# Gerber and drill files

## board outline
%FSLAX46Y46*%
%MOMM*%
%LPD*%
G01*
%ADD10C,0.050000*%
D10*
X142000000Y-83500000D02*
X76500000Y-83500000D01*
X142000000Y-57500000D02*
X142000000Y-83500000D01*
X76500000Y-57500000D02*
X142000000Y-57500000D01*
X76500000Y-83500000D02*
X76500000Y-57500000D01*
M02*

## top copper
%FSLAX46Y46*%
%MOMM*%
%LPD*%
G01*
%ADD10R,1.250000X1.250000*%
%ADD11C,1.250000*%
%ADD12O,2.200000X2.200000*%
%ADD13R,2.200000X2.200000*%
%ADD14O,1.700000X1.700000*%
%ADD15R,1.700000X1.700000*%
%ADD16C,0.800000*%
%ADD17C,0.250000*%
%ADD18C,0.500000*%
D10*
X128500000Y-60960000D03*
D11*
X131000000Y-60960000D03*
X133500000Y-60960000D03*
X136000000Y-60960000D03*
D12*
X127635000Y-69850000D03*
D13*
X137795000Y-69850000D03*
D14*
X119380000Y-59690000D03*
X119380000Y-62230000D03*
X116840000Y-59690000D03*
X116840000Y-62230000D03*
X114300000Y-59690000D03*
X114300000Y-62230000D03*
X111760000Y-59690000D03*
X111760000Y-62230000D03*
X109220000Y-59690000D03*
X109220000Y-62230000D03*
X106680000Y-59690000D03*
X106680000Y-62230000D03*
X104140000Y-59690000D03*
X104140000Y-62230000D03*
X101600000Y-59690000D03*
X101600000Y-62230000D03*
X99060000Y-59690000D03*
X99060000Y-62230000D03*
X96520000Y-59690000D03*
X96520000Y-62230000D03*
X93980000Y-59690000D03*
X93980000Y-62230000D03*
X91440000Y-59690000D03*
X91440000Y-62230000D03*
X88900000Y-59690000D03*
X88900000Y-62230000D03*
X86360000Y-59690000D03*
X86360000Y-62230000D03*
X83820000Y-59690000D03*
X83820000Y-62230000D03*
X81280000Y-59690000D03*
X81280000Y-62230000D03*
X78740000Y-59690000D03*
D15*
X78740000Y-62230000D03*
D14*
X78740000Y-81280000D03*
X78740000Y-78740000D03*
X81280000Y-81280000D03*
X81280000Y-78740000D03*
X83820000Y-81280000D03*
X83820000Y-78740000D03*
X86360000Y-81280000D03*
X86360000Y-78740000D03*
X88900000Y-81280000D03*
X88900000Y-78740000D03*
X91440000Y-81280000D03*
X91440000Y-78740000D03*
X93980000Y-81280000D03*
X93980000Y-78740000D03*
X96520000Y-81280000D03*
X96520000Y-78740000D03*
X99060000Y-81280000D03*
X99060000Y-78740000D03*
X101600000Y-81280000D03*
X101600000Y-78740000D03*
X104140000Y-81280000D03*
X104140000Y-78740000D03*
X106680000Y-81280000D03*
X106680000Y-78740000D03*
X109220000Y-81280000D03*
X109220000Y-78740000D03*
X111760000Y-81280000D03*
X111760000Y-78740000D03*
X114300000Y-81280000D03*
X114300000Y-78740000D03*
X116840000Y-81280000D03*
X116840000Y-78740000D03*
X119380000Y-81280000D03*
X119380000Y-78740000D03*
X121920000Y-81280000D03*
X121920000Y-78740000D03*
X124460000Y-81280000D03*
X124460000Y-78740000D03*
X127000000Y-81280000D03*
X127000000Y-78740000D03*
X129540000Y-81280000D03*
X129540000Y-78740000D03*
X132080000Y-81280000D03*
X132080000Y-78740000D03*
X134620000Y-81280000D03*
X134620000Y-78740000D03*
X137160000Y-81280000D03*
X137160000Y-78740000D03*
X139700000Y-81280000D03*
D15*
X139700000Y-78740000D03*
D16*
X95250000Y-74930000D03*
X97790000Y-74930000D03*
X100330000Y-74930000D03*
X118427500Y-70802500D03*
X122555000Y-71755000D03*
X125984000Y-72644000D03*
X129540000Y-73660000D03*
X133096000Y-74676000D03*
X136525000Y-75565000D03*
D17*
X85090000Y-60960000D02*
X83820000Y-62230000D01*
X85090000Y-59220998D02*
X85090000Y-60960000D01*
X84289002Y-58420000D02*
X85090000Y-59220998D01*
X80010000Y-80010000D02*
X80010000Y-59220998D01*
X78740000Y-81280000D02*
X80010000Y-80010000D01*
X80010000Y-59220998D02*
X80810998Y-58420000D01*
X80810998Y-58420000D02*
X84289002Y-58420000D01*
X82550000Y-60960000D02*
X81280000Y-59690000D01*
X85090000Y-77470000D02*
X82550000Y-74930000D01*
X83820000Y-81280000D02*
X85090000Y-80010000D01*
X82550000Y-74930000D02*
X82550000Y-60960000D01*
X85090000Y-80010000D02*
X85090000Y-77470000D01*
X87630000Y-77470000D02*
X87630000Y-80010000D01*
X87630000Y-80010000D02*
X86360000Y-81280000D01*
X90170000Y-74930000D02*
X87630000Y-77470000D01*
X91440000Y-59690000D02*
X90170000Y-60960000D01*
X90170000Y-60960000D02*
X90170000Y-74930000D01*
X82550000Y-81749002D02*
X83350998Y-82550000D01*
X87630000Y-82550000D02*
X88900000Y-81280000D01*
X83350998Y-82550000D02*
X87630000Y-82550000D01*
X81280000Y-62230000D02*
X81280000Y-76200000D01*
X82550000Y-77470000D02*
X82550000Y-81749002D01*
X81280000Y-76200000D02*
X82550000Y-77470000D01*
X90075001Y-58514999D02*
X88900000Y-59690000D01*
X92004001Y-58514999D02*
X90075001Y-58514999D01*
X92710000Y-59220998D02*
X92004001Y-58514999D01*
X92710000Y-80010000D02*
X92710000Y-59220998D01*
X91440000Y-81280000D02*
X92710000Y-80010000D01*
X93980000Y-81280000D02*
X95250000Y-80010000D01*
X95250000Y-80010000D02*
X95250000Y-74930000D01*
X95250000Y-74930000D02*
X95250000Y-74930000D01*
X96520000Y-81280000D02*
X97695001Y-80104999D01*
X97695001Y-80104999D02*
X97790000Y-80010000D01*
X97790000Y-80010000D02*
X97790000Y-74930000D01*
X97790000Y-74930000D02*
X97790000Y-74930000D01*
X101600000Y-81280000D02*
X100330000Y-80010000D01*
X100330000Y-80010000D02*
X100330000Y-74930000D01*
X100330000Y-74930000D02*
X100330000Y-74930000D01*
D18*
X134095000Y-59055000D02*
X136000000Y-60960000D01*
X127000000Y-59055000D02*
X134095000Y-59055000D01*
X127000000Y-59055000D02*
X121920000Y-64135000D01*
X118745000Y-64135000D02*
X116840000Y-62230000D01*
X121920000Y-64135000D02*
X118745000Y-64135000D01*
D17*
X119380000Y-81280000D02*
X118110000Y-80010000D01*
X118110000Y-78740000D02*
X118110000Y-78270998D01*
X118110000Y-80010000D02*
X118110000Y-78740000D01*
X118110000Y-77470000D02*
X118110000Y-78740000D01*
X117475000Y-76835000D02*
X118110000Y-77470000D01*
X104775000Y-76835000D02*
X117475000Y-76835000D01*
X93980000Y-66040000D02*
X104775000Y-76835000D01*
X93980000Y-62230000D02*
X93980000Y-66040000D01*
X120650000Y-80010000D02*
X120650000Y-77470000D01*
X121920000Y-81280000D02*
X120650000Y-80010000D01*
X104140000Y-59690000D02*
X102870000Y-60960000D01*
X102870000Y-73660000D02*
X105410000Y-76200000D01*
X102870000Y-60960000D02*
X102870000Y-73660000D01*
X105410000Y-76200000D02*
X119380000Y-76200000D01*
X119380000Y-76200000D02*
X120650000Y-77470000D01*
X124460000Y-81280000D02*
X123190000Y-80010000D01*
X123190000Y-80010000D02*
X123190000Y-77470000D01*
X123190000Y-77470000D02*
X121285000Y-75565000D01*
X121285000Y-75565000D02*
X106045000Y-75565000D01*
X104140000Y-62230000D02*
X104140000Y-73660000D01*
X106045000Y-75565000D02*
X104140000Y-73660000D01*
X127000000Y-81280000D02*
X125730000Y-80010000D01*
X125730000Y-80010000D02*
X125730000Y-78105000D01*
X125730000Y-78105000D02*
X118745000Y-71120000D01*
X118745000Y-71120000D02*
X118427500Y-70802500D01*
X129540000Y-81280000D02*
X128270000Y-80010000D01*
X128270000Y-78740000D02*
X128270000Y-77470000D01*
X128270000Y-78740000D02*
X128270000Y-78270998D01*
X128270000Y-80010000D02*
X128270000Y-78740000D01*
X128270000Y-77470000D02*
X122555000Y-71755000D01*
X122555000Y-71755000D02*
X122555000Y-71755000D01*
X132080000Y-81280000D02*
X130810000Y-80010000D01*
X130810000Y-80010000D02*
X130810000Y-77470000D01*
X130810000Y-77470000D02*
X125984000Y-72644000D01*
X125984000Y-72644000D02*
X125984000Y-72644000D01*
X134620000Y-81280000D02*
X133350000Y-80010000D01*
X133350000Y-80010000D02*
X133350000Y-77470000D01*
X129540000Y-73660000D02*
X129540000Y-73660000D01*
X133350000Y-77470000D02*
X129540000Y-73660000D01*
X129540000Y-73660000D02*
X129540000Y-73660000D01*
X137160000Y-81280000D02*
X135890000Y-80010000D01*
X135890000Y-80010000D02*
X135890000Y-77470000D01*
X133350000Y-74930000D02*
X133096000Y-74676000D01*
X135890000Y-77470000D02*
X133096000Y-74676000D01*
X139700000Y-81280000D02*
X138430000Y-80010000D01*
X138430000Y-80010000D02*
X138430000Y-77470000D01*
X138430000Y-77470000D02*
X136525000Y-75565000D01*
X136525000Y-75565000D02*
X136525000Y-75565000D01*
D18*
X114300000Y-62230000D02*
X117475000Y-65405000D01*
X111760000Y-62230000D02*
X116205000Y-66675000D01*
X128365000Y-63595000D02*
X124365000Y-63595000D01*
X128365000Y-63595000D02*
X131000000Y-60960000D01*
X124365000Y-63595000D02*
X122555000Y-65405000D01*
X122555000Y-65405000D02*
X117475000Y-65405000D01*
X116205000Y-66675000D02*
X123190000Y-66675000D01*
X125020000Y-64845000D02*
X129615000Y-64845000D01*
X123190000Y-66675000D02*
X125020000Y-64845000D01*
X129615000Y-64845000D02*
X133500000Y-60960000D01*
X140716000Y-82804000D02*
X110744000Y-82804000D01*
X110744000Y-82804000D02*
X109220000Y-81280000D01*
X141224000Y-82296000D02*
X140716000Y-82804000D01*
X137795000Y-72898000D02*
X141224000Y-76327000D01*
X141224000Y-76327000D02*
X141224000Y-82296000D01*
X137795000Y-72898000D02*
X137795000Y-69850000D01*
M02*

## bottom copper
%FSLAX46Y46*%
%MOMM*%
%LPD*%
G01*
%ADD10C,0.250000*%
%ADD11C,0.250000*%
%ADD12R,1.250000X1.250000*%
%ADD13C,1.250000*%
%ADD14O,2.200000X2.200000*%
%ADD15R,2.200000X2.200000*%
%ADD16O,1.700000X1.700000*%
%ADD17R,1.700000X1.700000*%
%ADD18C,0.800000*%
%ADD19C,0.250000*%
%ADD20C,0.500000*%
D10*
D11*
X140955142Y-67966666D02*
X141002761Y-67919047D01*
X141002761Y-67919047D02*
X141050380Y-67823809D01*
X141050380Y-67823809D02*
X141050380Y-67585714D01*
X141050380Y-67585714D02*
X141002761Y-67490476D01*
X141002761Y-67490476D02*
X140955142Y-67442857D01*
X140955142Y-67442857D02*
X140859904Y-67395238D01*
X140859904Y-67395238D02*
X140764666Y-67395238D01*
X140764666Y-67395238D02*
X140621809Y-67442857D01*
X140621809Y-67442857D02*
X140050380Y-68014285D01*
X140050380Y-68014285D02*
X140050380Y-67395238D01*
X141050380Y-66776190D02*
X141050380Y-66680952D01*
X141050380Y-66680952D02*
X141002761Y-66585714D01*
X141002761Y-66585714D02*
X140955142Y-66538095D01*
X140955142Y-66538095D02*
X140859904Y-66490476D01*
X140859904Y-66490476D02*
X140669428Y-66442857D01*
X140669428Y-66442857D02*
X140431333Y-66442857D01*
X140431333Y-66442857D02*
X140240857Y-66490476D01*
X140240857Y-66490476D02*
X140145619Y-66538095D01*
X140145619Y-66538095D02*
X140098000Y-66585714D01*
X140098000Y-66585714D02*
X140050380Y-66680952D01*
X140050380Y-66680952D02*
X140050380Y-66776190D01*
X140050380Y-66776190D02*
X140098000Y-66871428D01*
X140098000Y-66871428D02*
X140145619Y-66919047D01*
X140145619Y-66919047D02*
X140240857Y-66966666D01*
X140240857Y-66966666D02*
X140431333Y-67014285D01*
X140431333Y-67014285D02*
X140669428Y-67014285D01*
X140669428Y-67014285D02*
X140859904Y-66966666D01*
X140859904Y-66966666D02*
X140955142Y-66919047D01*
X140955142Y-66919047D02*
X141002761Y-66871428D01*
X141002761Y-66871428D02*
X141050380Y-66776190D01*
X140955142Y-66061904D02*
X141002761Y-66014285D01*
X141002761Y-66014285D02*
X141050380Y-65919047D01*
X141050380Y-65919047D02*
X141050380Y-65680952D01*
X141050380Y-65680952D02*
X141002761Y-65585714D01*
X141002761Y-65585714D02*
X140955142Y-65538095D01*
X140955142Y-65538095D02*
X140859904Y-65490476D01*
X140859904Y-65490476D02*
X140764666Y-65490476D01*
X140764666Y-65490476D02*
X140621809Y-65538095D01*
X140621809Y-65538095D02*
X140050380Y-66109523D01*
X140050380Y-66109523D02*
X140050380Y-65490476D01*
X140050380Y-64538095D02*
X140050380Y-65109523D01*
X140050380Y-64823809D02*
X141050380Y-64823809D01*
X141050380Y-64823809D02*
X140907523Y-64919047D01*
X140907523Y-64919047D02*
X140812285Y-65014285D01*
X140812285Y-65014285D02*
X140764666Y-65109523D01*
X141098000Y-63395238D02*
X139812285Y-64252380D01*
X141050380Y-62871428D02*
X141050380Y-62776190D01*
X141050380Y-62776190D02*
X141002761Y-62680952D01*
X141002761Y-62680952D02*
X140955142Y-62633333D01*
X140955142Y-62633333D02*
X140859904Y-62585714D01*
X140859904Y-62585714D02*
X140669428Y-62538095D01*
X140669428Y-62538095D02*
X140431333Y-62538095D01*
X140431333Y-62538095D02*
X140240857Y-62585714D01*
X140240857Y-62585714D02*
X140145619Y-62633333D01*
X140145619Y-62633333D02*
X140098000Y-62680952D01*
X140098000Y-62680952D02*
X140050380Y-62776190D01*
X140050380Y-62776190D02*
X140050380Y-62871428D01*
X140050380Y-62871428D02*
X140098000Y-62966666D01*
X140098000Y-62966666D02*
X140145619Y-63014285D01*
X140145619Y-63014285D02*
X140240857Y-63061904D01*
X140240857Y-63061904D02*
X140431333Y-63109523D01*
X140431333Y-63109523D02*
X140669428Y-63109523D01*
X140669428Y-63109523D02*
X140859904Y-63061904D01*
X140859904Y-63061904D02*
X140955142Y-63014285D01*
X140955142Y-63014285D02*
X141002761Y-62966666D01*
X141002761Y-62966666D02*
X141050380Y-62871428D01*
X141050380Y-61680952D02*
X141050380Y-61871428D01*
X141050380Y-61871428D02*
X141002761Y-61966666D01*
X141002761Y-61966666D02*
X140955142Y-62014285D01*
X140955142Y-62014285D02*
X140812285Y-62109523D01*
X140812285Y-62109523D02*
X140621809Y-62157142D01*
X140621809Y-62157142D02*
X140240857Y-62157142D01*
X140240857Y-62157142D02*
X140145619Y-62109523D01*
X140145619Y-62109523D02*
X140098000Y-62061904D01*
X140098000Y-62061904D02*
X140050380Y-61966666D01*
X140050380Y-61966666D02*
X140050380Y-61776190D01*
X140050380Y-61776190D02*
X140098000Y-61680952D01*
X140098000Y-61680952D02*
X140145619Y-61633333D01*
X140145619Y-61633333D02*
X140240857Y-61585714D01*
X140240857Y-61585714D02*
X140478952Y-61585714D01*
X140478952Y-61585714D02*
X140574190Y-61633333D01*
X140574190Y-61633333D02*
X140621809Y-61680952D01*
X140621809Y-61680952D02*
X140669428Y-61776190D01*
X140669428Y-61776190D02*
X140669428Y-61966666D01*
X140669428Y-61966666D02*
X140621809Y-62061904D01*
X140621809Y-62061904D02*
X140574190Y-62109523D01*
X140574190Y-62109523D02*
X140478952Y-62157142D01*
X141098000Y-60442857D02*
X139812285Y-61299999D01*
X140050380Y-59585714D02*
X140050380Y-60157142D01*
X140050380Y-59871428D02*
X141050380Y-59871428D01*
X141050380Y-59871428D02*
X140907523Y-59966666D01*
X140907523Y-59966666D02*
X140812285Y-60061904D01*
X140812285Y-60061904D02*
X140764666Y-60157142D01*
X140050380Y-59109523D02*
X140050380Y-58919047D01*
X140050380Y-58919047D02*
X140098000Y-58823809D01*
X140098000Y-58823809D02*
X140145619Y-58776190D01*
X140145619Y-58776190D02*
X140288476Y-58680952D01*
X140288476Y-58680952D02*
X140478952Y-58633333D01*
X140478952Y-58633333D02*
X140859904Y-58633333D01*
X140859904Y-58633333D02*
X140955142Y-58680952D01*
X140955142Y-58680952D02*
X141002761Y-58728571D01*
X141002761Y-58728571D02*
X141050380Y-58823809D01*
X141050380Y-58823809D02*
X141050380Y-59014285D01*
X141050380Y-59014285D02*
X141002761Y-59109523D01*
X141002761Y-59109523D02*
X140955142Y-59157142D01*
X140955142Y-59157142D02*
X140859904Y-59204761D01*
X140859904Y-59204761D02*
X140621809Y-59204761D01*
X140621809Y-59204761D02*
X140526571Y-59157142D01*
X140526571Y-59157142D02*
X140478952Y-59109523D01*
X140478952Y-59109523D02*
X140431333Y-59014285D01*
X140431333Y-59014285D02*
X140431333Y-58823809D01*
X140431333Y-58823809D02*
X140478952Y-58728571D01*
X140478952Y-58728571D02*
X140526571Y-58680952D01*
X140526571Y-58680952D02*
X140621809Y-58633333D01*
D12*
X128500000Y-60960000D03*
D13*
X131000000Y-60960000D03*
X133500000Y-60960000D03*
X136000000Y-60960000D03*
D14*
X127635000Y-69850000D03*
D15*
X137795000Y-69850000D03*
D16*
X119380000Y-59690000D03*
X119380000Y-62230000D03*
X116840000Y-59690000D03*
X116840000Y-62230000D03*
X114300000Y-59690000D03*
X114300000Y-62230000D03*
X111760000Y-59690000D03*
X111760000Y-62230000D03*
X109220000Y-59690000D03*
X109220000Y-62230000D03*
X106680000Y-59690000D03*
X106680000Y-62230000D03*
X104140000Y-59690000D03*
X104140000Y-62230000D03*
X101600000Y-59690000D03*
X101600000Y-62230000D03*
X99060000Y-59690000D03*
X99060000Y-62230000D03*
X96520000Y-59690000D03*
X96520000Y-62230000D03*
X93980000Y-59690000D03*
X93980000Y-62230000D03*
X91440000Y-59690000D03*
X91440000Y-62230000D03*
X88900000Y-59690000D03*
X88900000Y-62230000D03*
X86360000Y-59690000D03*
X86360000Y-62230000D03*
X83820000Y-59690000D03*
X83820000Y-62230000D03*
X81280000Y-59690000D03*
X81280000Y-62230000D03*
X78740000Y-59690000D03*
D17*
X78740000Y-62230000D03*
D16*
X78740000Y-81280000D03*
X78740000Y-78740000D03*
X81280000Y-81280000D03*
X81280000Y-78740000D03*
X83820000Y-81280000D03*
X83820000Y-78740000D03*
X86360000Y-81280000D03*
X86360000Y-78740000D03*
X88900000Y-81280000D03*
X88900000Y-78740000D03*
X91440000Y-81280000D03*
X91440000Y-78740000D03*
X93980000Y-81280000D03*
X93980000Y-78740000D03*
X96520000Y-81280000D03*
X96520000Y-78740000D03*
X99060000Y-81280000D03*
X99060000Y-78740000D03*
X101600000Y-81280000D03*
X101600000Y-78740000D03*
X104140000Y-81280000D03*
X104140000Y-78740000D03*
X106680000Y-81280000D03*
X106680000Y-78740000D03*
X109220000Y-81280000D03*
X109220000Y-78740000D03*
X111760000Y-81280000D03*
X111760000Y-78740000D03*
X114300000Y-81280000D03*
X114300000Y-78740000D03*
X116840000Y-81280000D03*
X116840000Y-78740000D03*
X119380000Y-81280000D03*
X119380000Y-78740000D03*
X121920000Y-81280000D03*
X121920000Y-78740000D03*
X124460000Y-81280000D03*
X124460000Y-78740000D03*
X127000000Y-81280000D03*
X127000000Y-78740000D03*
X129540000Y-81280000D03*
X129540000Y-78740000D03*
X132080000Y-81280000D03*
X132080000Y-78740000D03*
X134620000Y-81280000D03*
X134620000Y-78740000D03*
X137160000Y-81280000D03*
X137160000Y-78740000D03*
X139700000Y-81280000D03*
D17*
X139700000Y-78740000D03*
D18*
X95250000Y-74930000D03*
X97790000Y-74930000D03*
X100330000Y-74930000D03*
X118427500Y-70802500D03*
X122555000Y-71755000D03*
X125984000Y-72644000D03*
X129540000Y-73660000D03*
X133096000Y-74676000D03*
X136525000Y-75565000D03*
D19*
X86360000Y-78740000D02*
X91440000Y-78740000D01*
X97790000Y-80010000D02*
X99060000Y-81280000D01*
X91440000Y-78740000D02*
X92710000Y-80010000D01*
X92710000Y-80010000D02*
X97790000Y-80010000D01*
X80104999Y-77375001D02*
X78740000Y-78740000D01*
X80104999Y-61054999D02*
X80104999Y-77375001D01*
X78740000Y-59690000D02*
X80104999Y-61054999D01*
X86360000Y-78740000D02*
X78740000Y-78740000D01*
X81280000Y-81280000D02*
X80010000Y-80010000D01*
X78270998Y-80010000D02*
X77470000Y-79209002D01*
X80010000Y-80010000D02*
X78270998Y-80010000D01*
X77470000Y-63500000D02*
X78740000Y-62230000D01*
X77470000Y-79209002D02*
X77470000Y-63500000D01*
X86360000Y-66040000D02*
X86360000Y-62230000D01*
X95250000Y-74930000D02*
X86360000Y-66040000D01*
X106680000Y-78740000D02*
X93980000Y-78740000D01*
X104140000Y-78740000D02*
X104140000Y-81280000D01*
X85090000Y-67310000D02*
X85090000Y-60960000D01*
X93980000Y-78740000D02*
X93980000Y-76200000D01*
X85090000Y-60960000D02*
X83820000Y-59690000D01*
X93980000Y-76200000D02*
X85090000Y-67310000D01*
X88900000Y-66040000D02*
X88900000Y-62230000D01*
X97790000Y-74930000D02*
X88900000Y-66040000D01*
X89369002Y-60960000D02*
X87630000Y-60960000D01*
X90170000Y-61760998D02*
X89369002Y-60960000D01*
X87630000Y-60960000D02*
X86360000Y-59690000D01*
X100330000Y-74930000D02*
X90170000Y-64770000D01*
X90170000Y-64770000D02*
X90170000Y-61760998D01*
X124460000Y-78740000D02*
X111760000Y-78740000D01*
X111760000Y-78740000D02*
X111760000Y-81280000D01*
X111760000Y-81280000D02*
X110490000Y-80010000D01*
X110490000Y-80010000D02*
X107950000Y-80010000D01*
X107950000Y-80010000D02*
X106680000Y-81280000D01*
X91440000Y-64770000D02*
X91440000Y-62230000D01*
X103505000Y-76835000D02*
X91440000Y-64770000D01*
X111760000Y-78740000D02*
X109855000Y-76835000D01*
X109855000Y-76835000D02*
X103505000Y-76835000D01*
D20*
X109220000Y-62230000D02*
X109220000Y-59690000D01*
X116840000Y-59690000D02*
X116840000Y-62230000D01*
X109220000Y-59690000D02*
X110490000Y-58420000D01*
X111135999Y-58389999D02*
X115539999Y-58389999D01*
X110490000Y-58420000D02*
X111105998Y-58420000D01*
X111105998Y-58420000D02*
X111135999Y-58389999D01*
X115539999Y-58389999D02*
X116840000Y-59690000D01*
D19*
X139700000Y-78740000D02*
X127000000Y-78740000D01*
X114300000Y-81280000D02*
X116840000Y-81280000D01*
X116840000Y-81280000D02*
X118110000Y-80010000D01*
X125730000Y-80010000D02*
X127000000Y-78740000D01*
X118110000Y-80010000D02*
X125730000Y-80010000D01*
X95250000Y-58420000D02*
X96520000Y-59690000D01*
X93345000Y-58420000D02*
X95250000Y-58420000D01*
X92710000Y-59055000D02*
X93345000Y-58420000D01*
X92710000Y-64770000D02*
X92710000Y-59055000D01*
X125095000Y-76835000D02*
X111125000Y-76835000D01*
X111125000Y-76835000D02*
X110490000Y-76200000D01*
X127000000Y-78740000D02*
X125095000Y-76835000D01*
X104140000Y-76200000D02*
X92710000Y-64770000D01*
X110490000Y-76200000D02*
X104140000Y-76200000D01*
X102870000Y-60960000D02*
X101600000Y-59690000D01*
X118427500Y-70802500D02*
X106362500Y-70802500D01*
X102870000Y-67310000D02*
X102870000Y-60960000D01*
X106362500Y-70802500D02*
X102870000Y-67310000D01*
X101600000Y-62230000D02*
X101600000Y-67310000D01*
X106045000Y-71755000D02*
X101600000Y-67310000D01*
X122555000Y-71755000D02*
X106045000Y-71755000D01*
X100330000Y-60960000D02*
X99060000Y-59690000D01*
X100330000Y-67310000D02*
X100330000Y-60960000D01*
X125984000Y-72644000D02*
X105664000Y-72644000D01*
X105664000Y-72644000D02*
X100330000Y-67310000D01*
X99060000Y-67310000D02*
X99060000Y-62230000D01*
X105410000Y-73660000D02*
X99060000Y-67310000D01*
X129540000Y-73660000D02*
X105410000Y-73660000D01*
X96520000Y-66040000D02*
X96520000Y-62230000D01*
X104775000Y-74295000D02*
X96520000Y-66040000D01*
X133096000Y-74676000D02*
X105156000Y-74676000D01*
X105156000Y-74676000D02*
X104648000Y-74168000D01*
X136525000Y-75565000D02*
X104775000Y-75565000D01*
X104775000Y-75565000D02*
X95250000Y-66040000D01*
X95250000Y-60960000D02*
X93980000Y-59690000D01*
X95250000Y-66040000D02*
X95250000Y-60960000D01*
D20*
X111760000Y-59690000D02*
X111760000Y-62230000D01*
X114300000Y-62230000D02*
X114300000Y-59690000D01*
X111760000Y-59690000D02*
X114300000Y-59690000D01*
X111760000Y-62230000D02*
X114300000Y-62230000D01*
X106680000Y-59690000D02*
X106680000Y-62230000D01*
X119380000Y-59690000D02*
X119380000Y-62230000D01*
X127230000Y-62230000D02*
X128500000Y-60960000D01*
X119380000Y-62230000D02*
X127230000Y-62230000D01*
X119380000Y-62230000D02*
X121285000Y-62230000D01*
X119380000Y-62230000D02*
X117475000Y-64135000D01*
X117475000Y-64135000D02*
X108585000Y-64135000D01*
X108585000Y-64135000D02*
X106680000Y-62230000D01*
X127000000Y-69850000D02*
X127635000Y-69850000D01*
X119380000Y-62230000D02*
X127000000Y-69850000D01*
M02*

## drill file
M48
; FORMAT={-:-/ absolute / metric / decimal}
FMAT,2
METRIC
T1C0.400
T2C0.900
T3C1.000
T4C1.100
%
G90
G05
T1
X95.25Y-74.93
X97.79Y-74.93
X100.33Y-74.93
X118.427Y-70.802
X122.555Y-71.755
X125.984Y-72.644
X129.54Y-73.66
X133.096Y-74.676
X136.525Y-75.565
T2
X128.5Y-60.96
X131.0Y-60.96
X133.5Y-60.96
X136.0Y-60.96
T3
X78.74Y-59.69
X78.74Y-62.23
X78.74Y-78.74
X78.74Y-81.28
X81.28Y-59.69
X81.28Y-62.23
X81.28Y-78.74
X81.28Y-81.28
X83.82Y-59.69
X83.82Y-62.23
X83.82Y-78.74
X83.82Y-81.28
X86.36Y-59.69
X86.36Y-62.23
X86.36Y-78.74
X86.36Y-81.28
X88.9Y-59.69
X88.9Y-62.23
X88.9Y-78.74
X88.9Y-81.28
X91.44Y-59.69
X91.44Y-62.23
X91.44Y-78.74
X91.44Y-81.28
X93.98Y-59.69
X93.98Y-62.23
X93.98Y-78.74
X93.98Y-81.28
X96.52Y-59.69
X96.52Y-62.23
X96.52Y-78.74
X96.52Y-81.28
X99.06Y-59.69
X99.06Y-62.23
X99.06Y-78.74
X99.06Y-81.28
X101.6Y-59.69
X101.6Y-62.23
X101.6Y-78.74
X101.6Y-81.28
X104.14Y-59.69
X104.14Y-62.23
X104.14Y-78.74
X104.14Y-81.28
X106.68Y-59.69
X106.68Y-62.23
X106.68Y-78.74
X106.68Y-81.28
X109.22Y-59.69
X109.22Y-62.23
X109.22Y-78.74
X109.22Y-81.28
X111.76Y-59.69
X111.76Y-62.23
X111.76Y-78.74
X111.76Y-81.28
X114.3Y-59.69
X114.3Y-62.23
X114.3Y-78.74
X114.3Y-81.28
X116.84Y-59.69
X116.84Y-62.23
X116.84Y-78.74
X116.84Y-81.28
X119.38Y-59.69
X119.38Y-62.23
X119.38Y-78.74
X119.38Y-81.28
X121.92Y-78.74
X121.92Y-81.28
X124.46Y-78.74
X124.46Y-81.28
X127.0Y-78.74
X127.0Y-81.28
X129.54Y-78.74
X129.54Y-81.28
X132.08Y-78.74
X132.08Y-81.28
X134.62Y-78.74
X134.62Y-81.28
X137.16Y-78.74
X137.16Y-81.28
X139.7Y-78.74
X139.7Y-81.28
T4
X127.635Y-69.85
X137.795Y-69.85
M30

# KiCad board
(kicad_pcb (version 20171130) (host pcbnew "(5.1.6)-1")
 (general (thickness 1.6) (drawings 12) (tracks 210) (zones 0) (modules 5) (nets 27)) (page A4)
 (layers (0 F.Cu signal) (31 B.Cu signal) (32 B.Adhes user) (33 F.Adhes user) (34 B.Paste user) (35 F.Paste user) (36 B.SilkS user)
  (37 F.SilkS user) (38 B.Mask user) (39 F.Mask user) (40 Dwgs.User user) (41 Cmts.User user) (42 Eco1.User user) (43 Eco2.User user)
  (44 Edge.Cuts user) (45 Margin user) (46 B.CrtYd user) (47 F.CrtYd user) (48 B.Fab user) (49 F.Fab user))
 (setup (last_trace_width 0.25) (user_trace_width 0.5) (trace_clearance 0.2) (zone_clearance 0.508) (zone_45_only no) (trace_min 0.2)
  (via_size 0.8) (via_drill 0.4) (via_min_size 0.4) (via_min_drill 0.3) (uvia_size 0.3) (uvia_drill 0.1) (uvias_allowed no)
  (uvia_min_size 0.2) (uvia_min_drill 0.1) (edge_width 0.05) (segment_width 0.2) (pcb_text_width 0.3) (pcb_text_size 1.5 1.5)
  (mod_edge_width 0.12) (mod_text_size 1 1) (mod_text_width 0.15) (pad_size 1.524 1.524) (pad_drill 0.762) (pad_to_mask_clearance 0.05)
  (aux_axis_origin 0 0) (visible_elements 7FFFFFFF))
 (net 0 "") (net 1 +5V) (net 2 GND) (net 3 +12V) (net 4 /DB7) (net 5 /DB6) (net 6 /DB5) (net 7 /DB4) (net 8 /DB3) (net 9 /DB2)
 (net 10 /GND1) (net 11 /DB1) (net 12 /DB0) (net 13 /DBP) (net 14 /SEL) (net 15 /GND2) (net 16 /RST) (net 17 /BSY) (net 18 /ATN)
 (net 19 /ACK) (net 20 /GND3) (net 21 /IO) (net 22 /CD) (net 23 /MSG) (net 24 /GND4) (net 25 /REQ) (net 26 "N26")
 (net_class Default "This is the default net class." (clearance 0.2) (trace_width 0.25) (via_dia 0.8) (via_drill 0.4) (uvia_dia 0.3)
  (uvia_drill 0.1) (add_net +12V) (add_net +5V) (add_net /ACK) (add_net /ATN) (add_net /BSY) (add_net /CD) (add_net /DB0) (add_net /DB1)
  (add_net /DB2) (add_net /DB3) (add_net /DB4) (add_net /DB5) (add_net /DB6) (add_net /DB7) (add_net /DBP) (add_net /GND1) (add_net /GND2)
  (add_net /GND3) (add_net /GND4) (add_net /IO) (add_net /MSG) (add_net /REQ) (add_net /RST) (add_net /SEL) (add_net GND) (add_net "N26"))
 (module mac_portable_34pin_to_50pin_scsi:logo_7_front (layer F.Cu) (at 89.7 70.9)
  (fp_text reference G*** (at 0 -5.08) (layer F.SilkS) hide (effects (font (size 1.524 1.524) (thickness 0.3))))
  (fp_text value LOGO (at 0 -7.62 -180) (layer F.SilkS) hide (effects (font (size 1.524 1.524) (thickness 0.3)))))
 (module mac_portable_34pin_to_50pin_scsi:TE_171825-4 (layer F.Cu) (at 128.5 60.96)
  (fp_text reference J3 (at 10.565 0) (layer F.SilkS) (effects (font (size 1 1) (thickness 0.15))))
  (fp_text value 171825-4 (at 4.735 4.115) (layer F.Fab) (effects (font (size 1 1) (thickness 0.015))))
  (pad 1 thru_hole rect (at 0 0) (size 1.25 1.25) (drill 0.9) (layers *.Cu *.Mask) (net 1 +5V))
  (pad 2 thru_hole circle (at 2.5 0) (size 1.25 1.25) (drill 0.9) (layers *.Cu *.Mask) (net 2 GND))
  (pad 3 thru_hole circle (at 5 0) (size 1.25 1.25) (drill 0.9) (layers *.Cu *.Mask) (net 2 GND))
  (pad 4 thru_hole circle (at 7.5 0) (size 1.25 1.25) (drill 0.9) (layers *.Cu *.Mask) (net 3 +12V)))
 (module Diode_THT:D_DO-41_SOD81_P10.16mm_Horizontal (layer F.Cu) (at 137.795 69.85 180)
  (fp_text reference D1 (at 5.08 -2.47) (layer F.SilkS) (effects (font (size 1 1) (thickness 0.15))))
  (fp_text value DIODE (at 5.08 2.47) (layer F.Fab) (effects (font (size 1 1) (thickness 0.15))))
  (pad 2 thru_hole oval (at 10.16 0 180) (size 2.2 2.2) (drill 1.1) (layers *.Cu *.Mask) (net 1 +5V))
  (pad 1 thru_hole rect (at 0 0 180) (size 2.2 2.2) (drill 1.1) (layers *.Cu *.Mask) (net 1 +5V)))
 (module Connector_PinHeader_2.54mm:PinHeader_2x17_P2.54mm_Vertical (layer F.Cu) (at 78.74 62.23 90)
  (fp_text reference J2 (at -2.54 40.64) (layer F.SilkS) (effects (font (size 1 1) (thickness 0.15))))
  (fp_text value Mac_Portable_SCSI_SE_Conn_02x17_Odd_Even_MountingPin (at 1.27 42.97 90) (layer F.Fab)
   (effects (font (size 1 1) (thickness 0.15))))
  (pad 34 thru_hole oval (at 2.54 40.64 90) (size 1.7 1.7) (drill 1) (layers *.Cu *.Mask) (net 1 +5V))
  (pad 33 thru_hole oval (at 0 40.64 90) (size 1.7 1.7) (drill 1) (layers *.Cu *.Mask) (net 1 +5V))
  (pad 32 thru_hole oval (at 2.54 38.1 90) (size 1.7 1.7) (drill 1) (layers *.Cu *.Mask) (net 3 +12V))
  (pad 31 thru_hole oval (at 0 38.1 90) (size 1.7 1.7) (drill 1) (layers *.Cu *.Mask) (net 3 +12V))
  (pad 30 thru_hole oval (at 2.54 35.56 90) (size 1.7 1.7) (drill 1) (layers *.Cu *.Mask) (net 2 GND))
  (pad 29 thru_hole oval (at 0 35.56 90) (size 1.7 1.7) (drill 1) (layers *.Cu *.Mask) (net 2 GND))
  (pad 28 thru_hole oval (at 2.54 33.02 90) (size 1.7 1.7) (drill 1) (layers *.Cu *.Mask) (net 2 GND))
  (pad 27 thru_hole oval (at 0 33.02 90) (size 1.7 1.7) (drill 1) (layers *.Cu *.Mask) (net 2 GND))
  (pad 26 thru_hole oval (at 2.54 30.48 90) (size 1.7 1.7) (drill 1) (layers *.Cu *.Mask) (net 3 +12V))
  (pad 25 thru_hole oval (at 0 30.48 90) (size 1.7 1.7) (drill 1) (layers *.Cu *.Mask) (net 3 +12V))
  (pad 24 thru_hole oval (at 2.54 27.94 90) (size 1.7 1.7) (drill 1) (layers *.Cu *.Mask) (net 1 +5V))
  (pad 23 thru_hole oval (at 0 27.94 90) (size 1.7 1.7) (drill 1) (layers *.Cu *.Mask) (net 1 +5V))
  (pad 22 thru_hole oval (at 2.54 25.4 90) (size 1.7 1.7) (drill 1) (layers *.Cu *.Mask) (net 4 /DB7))
  (pad 21 thru_hole oval (at 0 25.4 90) (size 1.7 1.7) (drill 1) (layers *.Cu *.Mask) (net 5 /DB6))
  (pad 20 thru_hole oval (at 2.54 22.86 90) (size 1.7 1.7) (drill 1) (layers *.Cu *.Mask) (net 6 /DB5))
  (pad 19 thru_hole oval (at 0 22.86 90) (size 1.7 1.7) (drill 1) (layers *.Cu *.Mask) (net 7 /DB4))
  (pad 18 thru_hole oval (at 2.54 20.32 90) (size 1.7 1.7) (drill 1) (layers *.Cu *.Mask) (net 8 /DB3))
  (pad 17 thru_hole oval (at 0 20.32 90) (size 1.7 1.7) (drill 1) (layers *.Cu *.Mask) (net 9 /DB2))
  (pad 16 thru_hole oval (at 2.54 17.78 90) (size 1.7 1.7) (drill 1) (layers *.Cu *.Mask) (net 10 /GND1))
  (pad 15 thru_hole oval (at 0 17.78 90) (size 1.7 1.7) (drill 1) (layers *.Cu *.Mask) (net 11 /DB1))
  (pad 14 thru_hole oval (at 2.54 15.24 90) (size 1.7 1.7) (drill 1) (layers *.Cu *.Mask) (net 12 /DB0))
  (pad 13 thru_hole oval (at 0 15.24 90) (size 1.7 1.7) (drill 1) (layers *.Cu *.Mask) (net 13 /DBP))
  (pad 12 thru_hole oval (at 2.54 12.7 90) (size 1.7 1.7) (drill 1) (layers *.Cu *.Mask) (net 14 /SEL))
  (pad 11 thru_hole oval (at 0 12.7 90) (size 1.7 1.7) (drill 1) (layers *.Cu *.Mask) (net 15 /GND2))
  (pad 10 thru_hole oval (at 2.54 10.16 90) (size 1.7 1.7) (drill 1) (layers *.Cu *.Mask) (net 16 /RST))
  (pad 9 thru_hole oval (at 0 10.16 90) (size 1.7 1.7) (drill 1) (layers *.Cu *.Mask) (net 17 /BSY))
  (pad 8 thru_hole oval (at 2.54 7.62 90) (size 1.7 1.7) (drill 1) (layers *.Cu *.Mask) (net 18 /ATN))
  (pad 7 thru_hole oval (at 0 7.62 90) (size 1.7 1.7) (drill 1) (layers *.Cu *.Mask) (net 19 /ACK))
  (pad 6 thru_hole oval (at 2.54 5.08 90) (size 1.7 1.7) (drill 1) (layers *.Cu *.Mask) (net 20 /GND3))
  (pad 5 thru_hole oval (at 0 5.08 90) (size 1.7 1.7) (drill 1) (layers *.Cu *.Mask) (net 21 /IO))
  (pad 4 thru_hole oval (at 2.54 2.54 90) (size 1.7 1.7) (drill 1) (layers *.Cu *.Mask) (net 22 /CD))
  (pad 3 thru_hole oval (at 0 2.54 90) (size 1.7 1.7) (drill 1) (layers *.Cu *.Mask) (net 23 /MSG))
  (pad 2 thru_hole oval (at 2.54 0 90) (size 1.7 1.7) (drill 1) (layers *.Cu *.Mask) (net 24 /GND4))
  (pad 1 thru_hole rect (at 0 0 90) (size 1.7 1.7) (drill 1) (layers *.Cu *.Mask) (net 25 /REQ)))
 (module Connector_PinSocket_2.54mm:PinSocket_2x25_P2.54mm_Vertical (layer B.Cu) (at 139.7 78.74 90)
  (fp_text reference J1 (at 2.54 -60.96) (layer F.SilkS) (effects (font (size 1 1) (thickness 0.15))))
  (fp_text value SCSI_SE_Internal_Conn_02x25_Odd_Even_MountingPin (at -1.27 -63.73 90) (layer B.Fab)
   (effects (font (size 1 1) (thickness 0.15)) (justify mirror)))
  (pad 50 thru_hole oval (at -2.54 -60.96 90) (size 1.7 1.7) (drill 1) (layers *.Cu *.Mask) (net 21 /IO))
  (pad 49 thru_hole oval (at 0 -60.96 90) (size 1.7 1.7) (drill 1) (layers *.Cu *.Mask) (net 24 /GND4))
  (pad 48 thru_hole oval (at -2.54 -58.42 90) (size 1.7 1.7) (drill 1) (layers *.Cu *.Mask) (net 25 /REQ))
  (pad 47 thru_hole oval (at 0 -58.42 90) (size 1.7 1.7) (drill 1) (layers *.Cu *.Mask) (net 24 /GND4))
  (pad 46 thru_hole oval (at -2.54 -55.88 90) (size 1.7 1.7) (drill 1) (layers *.Cu *.Mask) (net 22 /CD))
  (pad 45 thru_hole oval (at 0 -55.88 90) (size 1.7 1.7) (drill 1) (layers *.Cu *.Mask) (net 24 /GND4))
  (pad 44 thru_hole oval (at -2.54 -53.34 90) (size 1.7 1.7) (drill 1) (layers *.Cu *.Mask) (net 14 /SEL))
  (pad 43 thru_hole oval (at 0 -53.34 90) (size 1.7 1.7) (drill 1) (layers *.Cu *.Mask) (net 24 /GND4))
  (pad 42 thru_hole oval (at -2.54 -50.8 90) (size 1.7 1.7) (drill 1) (layers *.Cu *.Mask) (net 23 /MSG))
  (pad 41 thru_hole oval (at 0 -50.8 90) (size 1.7 1.7) (drill 1) (layers *.Cu *.Mask) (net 24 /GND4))
  (pad 40 thru_hole oval (at -2.54 -48.26 90) (size 1.7 1.7) (drill 1) (layers *.Cu *.Mask) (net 16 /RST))
  (pad 39 thru_hole oval (at 0 -48.26 90) (size 1.7 1.7) (drill 1) (layers *.Cu *.Mask) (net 24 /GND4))
  (pad 38 thru_hole oval (at -2.54 -45.72 90) (size 1.7 1.7) (drill 1) (layers *.Cu *.Mask) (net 19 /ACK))
  (pad 37 thru_hole oval (at 0 -45.72 90) (size 1.7 1.7) (drill 1) (layers *.Cu *.Mask) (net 20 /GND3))
  (pad 36 thru_hole oval (at -2.54 -43.18 90) (size 1.7 1.7) (drill 1) (layers *.Cu *.Mask) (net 17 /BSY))
  (pad 35 thru_hole oval (at 0 -43.18 90) (size 1.7 1.7) (drill 1) (layers *.Cu *.Mask) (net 20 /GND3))
  (pad 34 thru_hole oval (at -2.54 -40.64 90) (size 1.7 1.7) (drill 1) (layers *.Cu *.Mask) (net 24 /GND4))
  (pad 33 thru_hole oval (at 0 -40.64 90) (size 1.7 1.7) (drill 1) (layers *.Cu *.Mask) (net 20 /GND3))
  (pad 32 thru_hole oval (at -2.54 -38.1 90) (size 1.7 1.7) (drill 1) (layers *.Cu *.Mask) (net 18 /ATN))
  (pad 31 thru_hole oval (at 0 -38.1 90) (size 1.7 1.7) (drill 1) (layers *.Cu *.Mask) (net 20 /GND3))
  (pad 30 thru_hole oval (at -2.54 -35.56 90) (size 1.7 1.7) (drill 1) (layers *.Cu *.Mask) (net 20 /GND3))
  (pad 29 thru_hole oval (at 0 -35.56 90) (size 1.7 1.7) (drill 1) (layers *.Cu *.Mask) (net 20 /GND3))
  (pad 28 thru_hole oval (at -2.54 -33.02 90) (size 1.7 1.7) (drill 1) (layers *.Cu *.Mask) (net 15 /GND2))
  (pad 27 thru_hole oval (at 0 -33.02 90) (size 1.7 1.7) (drill 1) (layers *.Cu *.Mask) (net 20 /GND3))
  (pad 26 thru_hole oval (at -2.54 -30.48 90) (size 1.7 1.7) (drill 1) (layers *.Cu *.Mask) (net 1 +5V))
  (pad 25 thru_hole oval (at 0 -30.48 90) (size 1.7 1.7) (drill 1) (layers *.Cu *.Mask) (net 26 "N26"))
  (pad 24 thru_hole oval (at -2.54 -27.94 90) (size 1.7 1.7) (drill 1) (layers *.Cu *.Mask) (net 15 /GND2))
  (pad 23 thru_hole oval (at 0 -27.94 90) (size 1.7 1.7) (drill 1) (layers *.Cu *.Mask) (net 15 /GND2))
  (pad 22 thru_hole oval (at -2.54 -25.4 90) (size 1.7 1.7) (drill 1) (layers *.Cu *.Mask) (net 10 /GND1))
  (pad 21 thru_hole oval (at 0 -25.4 90) (size 1.7 1.7) (drill 1) (layers *.Cu *.Mask) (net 15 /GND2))
  (pad 20 thru_hole oval (at -2.54 -22.86 90) (size 1.7 1.7) (drill 1) (layers *.Cu *.Mask) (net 10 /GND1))
  (pad 19 thru_hole oval (at 0 -22.86 90) (size 1.7 1.7) (drill 1) (layers *.Cu *.Mask) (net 15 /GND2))
  (pad 18 thru_hole oval (at -2.54 -20.32 90) (size 1.7 1.7) (drill 1) (layers *.Cu *.Mask) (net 13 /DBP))
  (pad 17 thru_hole oval (at 0 -20.32 90) (size 1.7 1.7) (drill 1) (layers *.Cu *.Mask) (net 15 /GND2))
  (pad 16 thru_hole oval (at -2.54 -17.78 90) (size 1.7 1.7) (drill 1) (layers *.Cu *.Mask) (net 4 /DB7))
  (pad 15 thru_hole oval (at 0 -17.78 90) (size 1.7 1.7) (drill 1) (layers *.Cu *.Mask) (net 15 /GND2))
  (pad 14 thru_hole oval (at -2.54 -15.24 90) (size 1.7 1.7) (drill 1) (layers *.Cu *.Mask) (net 5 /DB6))
  (pad 13 thru_hole oval (at 0 -15.24 90) (size 1.7 1.7) (drill 1) (layers *.Cu *.Mask) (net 15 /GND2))
  (pad 12 thru_hole oval (at -2.54 -12.7 90) (size 1.7 1.7) (drill 1) (layers *.Cu *.Mask) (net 6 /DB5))
  (pad 11 thru_hole oval (at 0 -12.7 90) (size 1.7 1.7) (drill 1) (layers *.Cu *.Mask) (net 10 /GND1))
  (pad 10 thru_hole oval (at -2.54 -10.16 90) (size 1.7 1.7) (drill 1) (layers *.Cu *.Mask) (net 7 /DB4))
  (pad 9 thru_hole oval (at 0 -10.16 90) (size 1.7 1.7) (drill 1) (layers *.Cu *.Mask) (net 10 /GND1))
  (pad 8 thru_hole oval (at -2.54 -7.62 90) (size 1.7 1.7) (drill 1) (layers *.Cu *.Mask) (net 8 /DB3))
  (pad 7 thru_hole oval (at 0 -7.62 90) (size 1.7 1.7) (drill 1) (layers *.Cu *.Mask) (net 10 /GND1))
  (pad 6 thru_hole oval (at -2.54 -5.08 90) (size 1.7 1.7) (drill 1) (layers *.Cu *.Mask) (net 9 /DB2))
  (pad 5 thru_hole oval (at 0 -5.08 90) (size 1.7 1.7) (drill 1) (layers *.Cu *.Mask) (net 10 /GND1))
  (pad 4 thru_hole oval (at -2.54 -2.54 90) (size 1.7 1.7) (drill 1) (layers *.Cu *.Mask) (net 11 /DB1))
  (pad 3 thru_hole oval (at 0 -2.54 90) (size 1.7 1.7) (drill 1) (layers *.Cu *.Mask) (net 10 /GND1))
  (pad 2 thru_hole oval (at -2.54 0 90) (size 1.7 1.7) (drill 1) (layers *.Cu *.Mask) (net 12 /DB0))
  (pad 1 thru_hole rect (at 0 0 90) (size 1.7 1.7) (drill 1) (layers *.Cu *.Mask) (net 10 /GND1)))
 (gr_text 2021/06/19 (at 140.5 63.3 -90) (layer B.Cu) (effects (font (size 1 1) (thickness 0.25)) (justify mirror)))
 (gr_line (start 142 83.5) (end 76.5 83.5) (layer Edge.Cuts) (width 0.05))
 (gr_line (start 142 57.5) (end 142 83.5) (layer Edge.Cuts) (width 0.05))
 (gr_line (start 76.5 57.5) (end 142 57.5) (layer Edge.Cuts) (width 0.05))
 (gr_line (start 76.5 83.5) (end 76.5 57.5) (layer Edge.Cuts) (width 0.05))
 (segment (start 85.09 60.96) (end 83.82 62.23) (width 0.25) (layer F.Cu) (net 21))
 (segment (start 85.09 59.220998) (end 85.09 60.96) (width 0.25) (layer F.Cu) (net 21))
 (segment (start 84.289002 58.42) (end 85.09 59.220998) (width 0.25) (layer F.Cu) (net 21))
 (segment (start 80.01 80.01) (end 80.01 59.220998) (width 0.25) (layer F.Cu) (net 21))
 (segment (start 78.74 81.28) (end 80.01 80.01) (width 0.25) (layer F.Cu) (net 21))
 (segment (start 80.01 59.220998) (end 80.810998 58.42) (width 0.25) (layer F.Cu) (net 21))
 (segment (start 80.810998 58.42) (end 84.289002 58.42) (width 0.25) (layer F.Cu) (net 21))
 (segment (start 86.36 78.74) (end 91.44 78.74) (width 0.25) (layer B.Cu) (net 24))
 (segment (start 97.79 80.01) (end 99.06 81.28) (width 0.25) (layer B.Cu) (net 24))
 (segment (start 91.44 78.74) (end 92.71 80.01) (width 0.25) (layer B.Cu) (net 24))
 (segment (start 92.71 80.01) (end 97.79 80.01) (width 0.25) (layer B.Cu) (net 24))
 (segment (start 80.104999 77.375001) (end 78.74 78.74) (width 0.25) (layer B.Cu) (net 24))
 (segment (start 80.104999 61.054999) (end 80.104999 77.375001) (width 0.25) (layer B.Cu) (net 24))
 (segment (start 78.74 59.69) (end 80.104999 61.054999) (width 0.25) (layer B.Cu) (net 24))
 (segment (start 86.36 78.74) (end 78.74 78.74) (width 0.25) (layer B.Cu) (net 24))
 (segment (start 81.28 81.28) (end 80.01 80.01) (width 0.25) (layer B.Cu) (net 25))
 (segment (start 78.270998 80.01) (end 77.47 79.209002) (width 0.25) (layer B.Cu) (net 25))
 (segment (start 80.01 80.01) (end 78.270998 80.01) (width 0.25) (layer B.Cu) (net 25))
 (segment (start 77.47 63.5) (end 78.74 62.23) (width 0.25) (layer B.Cu) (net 25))
 (segment (start 77.47 79.209002) (end 77.47 63.5) (width 0.25) (layer B.Cu) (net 25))
 (segment (start 82.55 60.96) (end 81.28 59.69) (width 0.25) (layer F.Cu) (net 22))
 (segment (start 85.09 77.47) (end 82.55 74.93) (width 0.25) (layer F.Cu) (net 22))
 (segment (start 83.82 81.28) (end 85.09 80.01) (width 0.25) (layer F.Cu) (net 22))
 (segment (start 82.55 74.93) (end 82.55 60.96) (width 0.25) (layer F.Cu) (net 22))
 (segment (start 85.09 80.01) (end 85.09 77.47) (width 0.25) (layer F.Cu) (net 22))
 (segment (start 87.63 77.47) (end 87.63 80.01) (width 0.25) (layer F.Cu) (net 14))
 (segment (start 87.63 80.01) (end 86.36 81.28) (width 0.25) (layer F.Cu) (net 14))
 (segment (start 90.17 74.93) (end 87.63 77.47) (width 0.25) (layer F.Cu) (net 14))
 (segment (start 91.44 59.69) (end 90.17 60.96) (width 0.25) (layer F.Cu) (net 14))
 (segment (start 90.17 60.96) (end 90.17 74.93) (width 0.25) (layer F.Cu) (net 14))
 (segment (start 82.55 81.749002) (end 83.350998 82.55) (width 0.25) (layer F.Cu) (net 23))
 (segment (start 87.63 82.55) (end 88.9 81.28) (width 0.25) (layer F.Cu) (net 23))
 (segment (start 83.350998 82.55) (end 87.63 82.55) (width 0.25) (layer F.Cu) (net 23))
 (segment (start 81.28 62.23) (end 81.28 76.2) (width 0.25) (layer F.Cu) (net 23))
 (segment (start 82.55 77.47) (end 82.55 81.749002) (width 0.25) (layer F.Cu) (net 23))
 (segment (start 81.28 76.2) (end 82.55 77.47) (width 0.25) (layer F.Cu) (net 23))
 (segment (start 90.075001 58.514999) (end 88.9 59.69) (width 0.25) (layer F.Cu) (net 16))
 (segment (start 92.004001 58.514999) (end 90.075001 58.514999) (width 0.25) (layer F.Cu) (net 16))
 (segment (start 92.71 59.220998) (end 92.004001 58.514999) (width 0.25) (layer F.Cu) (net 16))
 (segment (start 92.71 80.01) (end 92.71 59.220998) (width 0.25) (layer F.Cu) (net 16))
 (segment (start 91.44 81.28) (end 92.71 80.01) (width 0.25) (layer F.Cu) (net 16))
 (segment (start 93.98 81.28) (end 95.25 80.01) (width 0.25) (layer F.Cu) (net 19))
 (segment (start 95.25 80.01) (end 95.25 74.93) (width 0.25) (layer F.Cu) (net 19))
 (segment (start 95.25 74.93) (end 95.25 74.93) (width 0.25) (layer F.Cu) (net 19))
 (via (at 95.25 74.93) (size 0.8) (drill 0.4) (layers F.Cu B.Cu) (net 19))
 (segment (start 86.36 66.04) (end 86.36 62.23) (width 0.25) (layer B.Cu) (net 19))
 (segment (start 95.25 74.93) (end 86.36 66.04) (width 0.25) (layer B.Cu) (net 19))
 (segment (start 106.68 78.74) (end 93.98 78.74) (width 0.25) (layer B.Cu) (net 20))
 (segment (start 104.14 78.74) (end 104.14 81.28) (width 0.25) (layer B.Cu) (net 20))
 (segment (start 85.09 67.31) (end 85.09 60.96) (width 0.25) (layer B.Cu) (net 20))
 (segment (start 93.98 78.74) (end 93.98 76.2) (width 0.25) (layer B.Cu) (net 20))
 (segment (start 85.09 60.96) (end 83.82 59.69) (width 0.25) (layer B.Cu) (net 20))
 (segment (start 93.98 76.2) (end 85.09 67.31) (width 0.25) (layer B.Cu) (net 20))
 (segment (start 96.52 81.28) (end 97.695001 80.104999) (width 0.25) (layer F.Cu) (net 17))
 (segment (start 97.695001 80.104999) (end 97.79 80.01) (width 0.25) (layer F.Cu) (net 17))
 (segment (start 97.79 80.01) (end 97.79 74.93) (width 0.25) (layer F.Cu) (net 17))
 (segment (start 97.79 74.93) (end 97.79 74.93) (width 0.25) (layer F.Cu) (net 17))
 (via (at 97.79 74.93) (size 0.8) (drill 0.4) (layers F.Cu B.Cu) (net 17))
 (segment (start 88.9 66.04) (end 88.9 62.23) (width 0.25) (layer B.Cu) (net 17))
 (segment (start 97.79 74.93) (end 88.9 66.04) (width 0.25) (layer B.Cu) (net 17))
 (segment (start 101.6 81.28) (end 100.33 80.01) (width 0.25) (layer F.Cu) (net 18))
 (segment (start 100.33 80.01) (end 100.33 74.93) (width 0.25) (layer F.Cu) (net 18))
 (segment (start 100.33 74.93) (end 100.33 74.93) (width 0.25) (layer F.Cu) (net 18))
 (via (at 100.33 74.93) (size 0.8) (drill 0.4) (layers F.Cu B.Cu) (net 18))
 (segment (start 89.369002 60.96) (end 87.63 60.96) (width 0.25) (layer B.Cu) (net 18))
 (segment (start 90.17 61.760998) (end 89.369002 60.96) (width 0.25) (layer B.Cu) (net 18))
 (segment (start 87.63 60.96) (end 86.36 59.69) (width 0.25) (layer B.Cu) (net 18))
 (segment (start 100.33 74.93) (end 90.17 64.77) (width 0.25) (layer B.Cu) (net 18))
 (segment (start 90.17 64.77) (end 90.17 61.760998) (width 0.25) (layer B.Cu) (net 18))
 (segment (start 124.46 78.74) (end 111.76 78.74) (width 0.25) (layer B.Cu) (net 15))
 (segment (start 111.76 78.74) (end 111.76 81.28) (width 0.25) (layer B.Cu) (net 15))
 (segment (start 111.76 81.28) (end 110.49 80.01) (width 0.25) (layer B.Cu) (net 15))
 (segment (start 110.49 80.01) (end 107.95 80.01) (width 0.25) (layer B.Cu) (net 15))
 (segment (start 107.95 80.01) (end 106.68 81.28) (width 0.25) (layer B.Cu) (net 15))
 (segment (start 91.44 64.77) (end 91.44 62.23) (width 0.25) (layer B.Cu) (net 15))
 (segment (start 103.505 76.835) (end 91.44 64.77) (width 0.25) (layer B.Cu) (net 15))
 (segment (start 111.76 78.74) (end 109.855 76.835) (width 0.25) (layer B.Cu) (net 15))
 (segment (start 109.855 76.835) (end 103.505 76.835) (width 0.25) (layer B.Cu) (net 15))
 (segment (start 109.22 62.23) (end 109.22 59.69) (width 0.5) (layer B.Cu) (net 3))
 (segment (start 116.84 59.69) (end 116.84 62.23) (width 0.5) (layer B.Cu) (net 3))
 (segment (start 109.22 59.69) (end 110.49 58.42) (width 0.5) (layer B.Cu) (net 3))
 (segment (start 111.135999 58.389999) (end 115.539999 58.389999) (width 0.5) (layer B.Cu) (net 3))
 (segment (start 110.49 58.42) (end 111.105998 58.42) (width 0.5) (layer B.Cu) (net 3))
 (segment (start 111.105998 58.42) (end 111.135999 58.389999) (width 0.5) (layer B.Cu) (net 3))
 (segment (start 115.539999 58.389999) (end 116.84 59.69) (width 0.5) (layer B.Cu) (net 3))
 (segment (start 134.095 59.055) (end 136 60.96) (width 0.5) (layer F.Cu) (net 3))
 (segment (start 127 59.055) (end 134.095 59.055) (width 0.5) (layer F.Cu) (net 3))
 (segment (start 127 59.055) (end 121.92 64.135) (width 0.5) (layer F.Cu) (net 3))
 (segment (start 118.745 64.135) (end 116.84 62.23) (width 0.5) (layer F.Cu) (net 3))
 (segment (start 121.92 64.135) (end 118.745 64.135) (width 0.5) (layer F.Cu) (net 3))
 (segment (start 139.7 78.74) (end 127 78.74) (width 0.25) (layer B.Cu) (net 10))
 (segment (start 114.3 81.28) (end 116.84 81.28) (width 0.25) (layer B.Cu) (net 10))
 (segment (start 116.84 81.28) (end 118.11 80.01) (width 0.25) (layer B.Cu) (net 10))
 (segment (start 125.73 80.01) (end 127 78.74) (width 0.25) (layer B.Cu) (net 10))
 (segment (start 118.11 80.01) (end 125.73 80.01) (width 0.25) (layer B.Cu) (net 10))
 (segment (start 95.25 58.42) (end 96.52 59.69) (width 0.25) (layer B.Cu) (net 10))
 (segment (start 93.345 58.42) (end 95.25 58.42) (width 0.25) (layer B.Cu) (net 10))
 (segment (start 92.71 59.055) (end 93.345 58.42) (width 0.25) (layer B.Cu) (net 10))
 (segment (start 92.71 64.77) (end 92.71 59.055) (width 0.25) (layer B.Cu) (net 10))
 (segment (start 125.095 76.835) (end 111.125 76.835) (width 0.25) (layer B.Cu) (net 10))
 (segment (start 111.125 76.835) (end 110.49 76.2) (width 0.25) (layer B.Cu) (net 10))
 (segment (start 127 78.74) (end 125.095 76.835) (width 0.25) (layer B.Cu) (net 10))
 (segment (start 104.14 76.2) (end 92.71 64.77) (width 0.25) (layer B.Cu) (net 10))
 (segment (start 110.49 76.2) (end 104.14 76.2) (width 0.25) (layer B.Cu) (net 10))
 (segment (start 119.38 81.28) (end 118.11 80.01) (width 0.25) (layer F.Cu) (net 13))
 (segment (start 118.11 78.74) (end 118.11 78.270998) (width 0.25) (layer F.Cu) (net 13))
 (segment (start 118.11 80.01) (end 118.11 78.74) (width 0.25) (layer F.Cu) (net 13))
 (segment (start 118.11 77.47) (end 118.11 78.74) (width 0.25) (layer F.Cu) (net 13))
 (segment (start 117.475 76.835) (end 118.11 77.47) (width 0.25) (layer F.Cu) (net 13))
 (segment (start 104.775 76.835) (end 117.475 76.835) (width 0.25) (layer F.Cu) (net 13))
 (segment (start 93.98 66.04) (end 104.775 76.835) (width 0.25) (layer F.Cu) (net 13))
 (segment (start 93.98 62.23) (end 93.98 66.04) (width 0.25) (layer F.Cu) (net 13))
 (segment (start 120.65 80.01) (end 120.65 77.47) (width 0.25) (layer F.Cu) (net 4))
 (segment (start 121.92 81.28) (end 120.65 80.01) (width 0.25) (layer F.Cu) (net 4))
 (segment (start 104.14 59.69) (end 102.87 60.96) (width 0.25) (layer F.Cu) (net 4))
 (segment (start 102.87 73.66) (end 105.41 76.2) (width 0.25) (layer F.Cu) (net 4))
 (segment (start 102.87 60.96) (end 102.87 73.66) (width 0.25) (layer F.Cu) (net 4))
 (segment (start 105.41 76.2) (end 119.38 76.2) (width 0.25) (layer F.Cu) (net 4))
 (segment (start 119.38 76.2) (end 120.65 77.47) (width 0.25) (layer F.Cu) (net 4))
 (segment (start 124.46 81.28) (end 123.19 80.01) (width 0.25) (layer F.Cu) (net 5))
 (segment (start 123.19 80.01) (end 123.19 77.47) (width 0.25) (layer F.Cu) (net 5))
 (segment (start 123.19 77.47) (end 121.285 75.565) (width 0.25) (layer F.Cu) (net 5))
 (segment (start 121.285 75.565) (end 106.045 75.565) (width 0.25) (layer F.Cu) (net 5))
 (segment (start 104.14 62.23) (end 104.14 73.66) (width 0.25) (layer F.Cu) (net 5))
 (segment (start 106.045 75.565) (end 104.14 73.66) (width 0.25) (layer F.Cu) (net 5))
 (segment (start 127 81.28) (end 125.73 80.01) (width 0.25) (layer F.Cu) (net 6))
 (segment (start 125.73 80.01) (end 125.73 78.105) (width 0.25) (layer F.Cu) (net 6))
 (segment (start 125.73 78.105) (end 118.745 71.12) (width 0.25) (layer F.Cu) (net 6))
 (segment (start 118.745 71.12) (end 118.4275 70.8025) (width 0.25) (layer F.Cu) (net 6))
 (via (at 118.4275 70.8025) (size 0.8) (drill 0.4) (layers F.Cu B.Cu) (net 6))
 (segment (start 102.87 60.96) (end 101.6 59.69) (width 0.25) (layer B.Cu) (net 6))
 (segment (start 118.4275 70.8025) (end 106.3625 70.8025) (width 0.25) (layer B.Cu) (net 6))
 (segment (start 102.87 67.31) (end 102.87 60.96) (width 0.25) (layer B.Cu) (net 6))
 (segment (start 106.3625 70.8025) (end 102.87 67.31) (width 0.25) (layer B.Cu) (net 6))
 (segment (start 129.54 81.28) (end 128.27 80.01) (width 0.25) (layer F.Cu) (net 7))
 (segment (start 128.27 78.74) (end 128.27 77.47) (width 0.25) (layer F.Cu) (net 7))
 (segment (start 128.27 78.74) (end 128.27 78.270998) (width 0.25) (layer F.Cu) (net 7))
 (segment (start 128.27 80.01) (end 128.27 78.74) (width 0.25) (layer F.Cu) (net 7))
 (segment (start 101.6 62.23) (end 101.6 67.31) (width 0.25) (layer B.Cu) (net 7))
 (segment (start 128.27 77.47) (end 122.555 71.755) (width 0.25) (layer F.Cu) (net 7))
 (segment (start 122.555 71.755) (end 122.555 71.755) (width 0.25) (layer F.Cu) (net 7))
 (via (at 122.555 71.755) (size 0.8) (drill 0.4) (layers F.Cu B.Cu) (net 7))
 (segment (start 106.045 71.755) (end 101.6 67.31) (width 0.25) (layer B.Cu) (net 7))
 (segment (start 122.555 71.755) (end 106.045 71.755) (width 0.25) (layer B.Cu) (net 7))
 (segment (start 132.08 81.28) (end 130.81 80.01) (width 0.25) (layer F.Cu) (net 8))
 (segment (start 130.81 80.01) (end 130.81 77.47) (width 0.25) (layer F.Cu) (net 8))
 (segment (start 130.81 77.47) (end 125.984 72.644) (width 0.25) (layer F.Cu) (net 8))
 (segment (start 125.984 72.644) (end 125.984 72.644) (width 0.25) (layer F.Cu) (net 8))
 (via (at 125.984 72.644) (size 0.8) (drill 0.4) (layers F.Cu B.Cu) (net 8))
 (segment (start 100.33 60.96) (end 99.06 59.69) (width 0.25) (layer B.Cu) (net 8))
 (segment (start 100.33 67.31) (end 100.33 60.96) (width 0.25) (layer B.Cu) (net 8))
 (segment (start 125.984 72.644) (end 105.664 72.644) (width 0.25) (layer B.Cu) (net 8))
 (segment (start 105.664 72.644) (end 100.33 67.31) (width 0.25) (layer B.Cu) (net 8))
 (segment (start 134.62 81.28) (end 133.35 80.01) (width 0.25) (layer F.Cu) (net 9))
 (segment (start 133.35 80.01) (end 133.35 77.47) (width 0.25) (layer F.Cu) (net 9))
 (segment (start 129.54 73.66) (end 129.54 73.66) (width 0.25) (layer F.Cu) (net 9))
 (segment (start 99.06 67.31) (end 99.06 62.23) (width 0.25) (layer B.Cu) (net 9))
 (segment (start 105.41 73.66) (end 99.06 67.31) (width 0.25) (layer B.Cu) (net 9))
 (segment (start 133.35 77.47) (end 129.54 73.66) (width 0.25) (layer F.Cu) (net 9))
 (segment (start 129.54 73.66) (end 129.54 73.66) (width 0.25) (layer F.Cu) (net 9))
 (via (at 129.54 73.66) (size 0.8) (drill 0.4) (layers F.Cu B.Cu) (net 9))
 (segment (start 129.54 73.66) (end 105.41 73.66) (width 0.25) (layer B.Cu) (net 9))
 (segment (start 137.16 81.28) (end 135.89 80.01) (width 0.25) (layer F.Cu) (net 11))
 (segment (start 135.89 80.01) (end 135.89 77.47) (width 0.25) (layer F.Cu) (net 11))
 (segment (start 96.52 66.04) (end 96.52 62.23) (width 0.25) (layer B.Cu) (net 11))
 (segment (start 104.775 74.295) (end 96.52 66.04) (width 0.25) (layer B.Cu) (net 11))
 (segment (start 133.096 74.676) (end 105.156 74.676) (width 0.25) (layer B.Cu) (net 11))
 (segment (start 105.156 74.676) (end 104.648 74.168) (width 0.25) (layer B.Cu) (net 11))
 (segment (start 133.35 74.93) (end 133.096 74.676) (width 0.25) (layer F.Cu) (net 11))
 (via (at 133.096 74.676) (size 0.8) (drill 0.4) (layers F.Cu B.Cu) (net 11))
 (segment (start 135.89 77.47) (end 133.096 74.676) (width 0.25) (layer F.Cu) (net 11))
 (segment (start 139.7 81.28) (end 138.43 80.01) (width 0.25) (layer F.Cu) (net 12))
 (segment (start 138.43 80.01) (end 138.43 77.47) (width 0.25) (layer F.Cu) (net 12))
 (segment (start 138.43 77.47) (end 136.525 75.565) (width 0.25) (layer F.Cu) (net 12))
 (segment (start 136.525 75.565) (end 136.525 75.565) (width 0.25) (layer F.Cu) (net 12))
 (via (at 136.525 75.565) (size 0.8) (drill 0.4) (layers F.Cu B.Cu) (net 12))
 (segment (start 136.525 75.565) (end 104.775 75.565) (width 0.25) (layer B.Cu) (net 12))
 (segment (start 104.775 75.565) (end 95.25 66.04) (width 0.25) (layer B.Cu) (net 12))
 (segment (start 95.25 60.96) (end 93.98 59.69) (width 0.25) (layer B.Cu) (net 12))
 (segment (start 95.25 66.04) (end 95.25 60.96) (width 0.25) (layer B.Cu) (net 12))
 (segment (start 111.76 59.69) (end 111.76 62.23) (width 0.5) (layer B.Cu) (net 2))
 (segment (start 114.3 62.23) (end 114.3 59.69) (width 0.5) (layer B.Cu) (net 2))
 (segment (start 111.76 59.69) (end 114.3 59.69) (width 0.5) (layer B.Cu) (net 2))
 (segment (start 111.76 62.23) (end 114.3 62.23) (width 0.5) (layer B.Cu) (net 2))
 (segment (start 114.3 62.23) (end 117.475 65.405) (width 0.5) (layer F.Cu) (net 2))
 (segment (start 111.76 62.23) (end 116.205 66.675) (width 0.5) (layer F.Cu) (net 2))
 (segment (start 128.365 63.595) (end 124.365 63.595) (width 0.5) (layer F.Cu) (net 2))
 (segment (start 128.365 63.595) (end 131 60.96) (width 0.5) (layer F.Cu) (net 2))
 (segment (start 124.365 63.595) (end 122.555 65.405) (width 0.5) (layer F.Cu) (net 2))
 (segment (start 122.555 65.405) (end 117.475 65.405) (width 0.5) (layer F.Cu) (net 2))
 (segment (start 116.205 66.675) (end 123.19 66.675) (width 0.5) (layer F.Cu) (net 2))
 (segment (start 125.02 64.845) (end 129.615 64.845) (width 0.5) (layer F.Cu) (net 2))
 (segment (start 123.19 66.675) (end 125.02 64.845) (width 0.5) (layer F.Cu) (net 2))
 (segment (start 129.615 64.845) (end 133.5 60.96) (width 0.5) (layer F.Cu) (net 2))
 (segment (start 106.68 59.69) (end 106.68 62.23) (width 0.5) (layer B.Cu) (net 1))
 (segment (start 119.38 59.69) (end 119.38 62.23) (width 0.5) (layer B.Cu) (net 1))
 (segment (start 127.23 62.23) (end 128.5 60.96) (width 0.5) (layer B.Cu) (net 1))
 (segment (start 119.38 62.23) (end 127.23 62.23) (width 0.5) (layer B.Cu) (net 1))
 (segment (start 119.38 62.23) (end 121.285 62.23) (width 0.5) (layer B.Cu) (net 1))
 (segment (start 119.38 62.23) (end 117.475 64.135) (width 0.5) (layer B.Cu) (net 1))
 (segment (start 117.475 64.135) (end 108.585 64.135) (width 0.5) (layer B.Cu) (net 1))
 (segment (start 108.585 64.135) (end 106.68 62.23) (width 0.5) (layer B.Cu) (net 1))
 (segment (start 140.716 82.804) (end 110.744 82.804) (width 0.5) (layer F.Cu) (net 1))
 (segment (start 110.744 82.804) (end 109.22 81.28) (width 0.5) (layer F.Cu) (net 1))
 (segment (start 141.224 82.296) (end 140.716 82.804) (width 0.5) (layer F.Cu) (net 1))
 (segment (start 137.795 72.898) (end 141.224 76.327) (width 0.5) (layer F.Cu) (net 1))
 (segment (start 141.224 76.327) (end 141.224 82.296) (width 0.5) (layer F.Cu) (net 1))
 (segment (start 127 69.85) (end 127.635 69.85) (width 0.5) (layer B.Cu) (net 1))
 (segment (start 119.38 62.23) (end 127 69.85) (width 0.5) (layer B.Cu) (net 1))
 (segment (start 137.795 72.898) (end 137.795 69.85) (width 0.5) (layer F.Cu) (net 1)))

